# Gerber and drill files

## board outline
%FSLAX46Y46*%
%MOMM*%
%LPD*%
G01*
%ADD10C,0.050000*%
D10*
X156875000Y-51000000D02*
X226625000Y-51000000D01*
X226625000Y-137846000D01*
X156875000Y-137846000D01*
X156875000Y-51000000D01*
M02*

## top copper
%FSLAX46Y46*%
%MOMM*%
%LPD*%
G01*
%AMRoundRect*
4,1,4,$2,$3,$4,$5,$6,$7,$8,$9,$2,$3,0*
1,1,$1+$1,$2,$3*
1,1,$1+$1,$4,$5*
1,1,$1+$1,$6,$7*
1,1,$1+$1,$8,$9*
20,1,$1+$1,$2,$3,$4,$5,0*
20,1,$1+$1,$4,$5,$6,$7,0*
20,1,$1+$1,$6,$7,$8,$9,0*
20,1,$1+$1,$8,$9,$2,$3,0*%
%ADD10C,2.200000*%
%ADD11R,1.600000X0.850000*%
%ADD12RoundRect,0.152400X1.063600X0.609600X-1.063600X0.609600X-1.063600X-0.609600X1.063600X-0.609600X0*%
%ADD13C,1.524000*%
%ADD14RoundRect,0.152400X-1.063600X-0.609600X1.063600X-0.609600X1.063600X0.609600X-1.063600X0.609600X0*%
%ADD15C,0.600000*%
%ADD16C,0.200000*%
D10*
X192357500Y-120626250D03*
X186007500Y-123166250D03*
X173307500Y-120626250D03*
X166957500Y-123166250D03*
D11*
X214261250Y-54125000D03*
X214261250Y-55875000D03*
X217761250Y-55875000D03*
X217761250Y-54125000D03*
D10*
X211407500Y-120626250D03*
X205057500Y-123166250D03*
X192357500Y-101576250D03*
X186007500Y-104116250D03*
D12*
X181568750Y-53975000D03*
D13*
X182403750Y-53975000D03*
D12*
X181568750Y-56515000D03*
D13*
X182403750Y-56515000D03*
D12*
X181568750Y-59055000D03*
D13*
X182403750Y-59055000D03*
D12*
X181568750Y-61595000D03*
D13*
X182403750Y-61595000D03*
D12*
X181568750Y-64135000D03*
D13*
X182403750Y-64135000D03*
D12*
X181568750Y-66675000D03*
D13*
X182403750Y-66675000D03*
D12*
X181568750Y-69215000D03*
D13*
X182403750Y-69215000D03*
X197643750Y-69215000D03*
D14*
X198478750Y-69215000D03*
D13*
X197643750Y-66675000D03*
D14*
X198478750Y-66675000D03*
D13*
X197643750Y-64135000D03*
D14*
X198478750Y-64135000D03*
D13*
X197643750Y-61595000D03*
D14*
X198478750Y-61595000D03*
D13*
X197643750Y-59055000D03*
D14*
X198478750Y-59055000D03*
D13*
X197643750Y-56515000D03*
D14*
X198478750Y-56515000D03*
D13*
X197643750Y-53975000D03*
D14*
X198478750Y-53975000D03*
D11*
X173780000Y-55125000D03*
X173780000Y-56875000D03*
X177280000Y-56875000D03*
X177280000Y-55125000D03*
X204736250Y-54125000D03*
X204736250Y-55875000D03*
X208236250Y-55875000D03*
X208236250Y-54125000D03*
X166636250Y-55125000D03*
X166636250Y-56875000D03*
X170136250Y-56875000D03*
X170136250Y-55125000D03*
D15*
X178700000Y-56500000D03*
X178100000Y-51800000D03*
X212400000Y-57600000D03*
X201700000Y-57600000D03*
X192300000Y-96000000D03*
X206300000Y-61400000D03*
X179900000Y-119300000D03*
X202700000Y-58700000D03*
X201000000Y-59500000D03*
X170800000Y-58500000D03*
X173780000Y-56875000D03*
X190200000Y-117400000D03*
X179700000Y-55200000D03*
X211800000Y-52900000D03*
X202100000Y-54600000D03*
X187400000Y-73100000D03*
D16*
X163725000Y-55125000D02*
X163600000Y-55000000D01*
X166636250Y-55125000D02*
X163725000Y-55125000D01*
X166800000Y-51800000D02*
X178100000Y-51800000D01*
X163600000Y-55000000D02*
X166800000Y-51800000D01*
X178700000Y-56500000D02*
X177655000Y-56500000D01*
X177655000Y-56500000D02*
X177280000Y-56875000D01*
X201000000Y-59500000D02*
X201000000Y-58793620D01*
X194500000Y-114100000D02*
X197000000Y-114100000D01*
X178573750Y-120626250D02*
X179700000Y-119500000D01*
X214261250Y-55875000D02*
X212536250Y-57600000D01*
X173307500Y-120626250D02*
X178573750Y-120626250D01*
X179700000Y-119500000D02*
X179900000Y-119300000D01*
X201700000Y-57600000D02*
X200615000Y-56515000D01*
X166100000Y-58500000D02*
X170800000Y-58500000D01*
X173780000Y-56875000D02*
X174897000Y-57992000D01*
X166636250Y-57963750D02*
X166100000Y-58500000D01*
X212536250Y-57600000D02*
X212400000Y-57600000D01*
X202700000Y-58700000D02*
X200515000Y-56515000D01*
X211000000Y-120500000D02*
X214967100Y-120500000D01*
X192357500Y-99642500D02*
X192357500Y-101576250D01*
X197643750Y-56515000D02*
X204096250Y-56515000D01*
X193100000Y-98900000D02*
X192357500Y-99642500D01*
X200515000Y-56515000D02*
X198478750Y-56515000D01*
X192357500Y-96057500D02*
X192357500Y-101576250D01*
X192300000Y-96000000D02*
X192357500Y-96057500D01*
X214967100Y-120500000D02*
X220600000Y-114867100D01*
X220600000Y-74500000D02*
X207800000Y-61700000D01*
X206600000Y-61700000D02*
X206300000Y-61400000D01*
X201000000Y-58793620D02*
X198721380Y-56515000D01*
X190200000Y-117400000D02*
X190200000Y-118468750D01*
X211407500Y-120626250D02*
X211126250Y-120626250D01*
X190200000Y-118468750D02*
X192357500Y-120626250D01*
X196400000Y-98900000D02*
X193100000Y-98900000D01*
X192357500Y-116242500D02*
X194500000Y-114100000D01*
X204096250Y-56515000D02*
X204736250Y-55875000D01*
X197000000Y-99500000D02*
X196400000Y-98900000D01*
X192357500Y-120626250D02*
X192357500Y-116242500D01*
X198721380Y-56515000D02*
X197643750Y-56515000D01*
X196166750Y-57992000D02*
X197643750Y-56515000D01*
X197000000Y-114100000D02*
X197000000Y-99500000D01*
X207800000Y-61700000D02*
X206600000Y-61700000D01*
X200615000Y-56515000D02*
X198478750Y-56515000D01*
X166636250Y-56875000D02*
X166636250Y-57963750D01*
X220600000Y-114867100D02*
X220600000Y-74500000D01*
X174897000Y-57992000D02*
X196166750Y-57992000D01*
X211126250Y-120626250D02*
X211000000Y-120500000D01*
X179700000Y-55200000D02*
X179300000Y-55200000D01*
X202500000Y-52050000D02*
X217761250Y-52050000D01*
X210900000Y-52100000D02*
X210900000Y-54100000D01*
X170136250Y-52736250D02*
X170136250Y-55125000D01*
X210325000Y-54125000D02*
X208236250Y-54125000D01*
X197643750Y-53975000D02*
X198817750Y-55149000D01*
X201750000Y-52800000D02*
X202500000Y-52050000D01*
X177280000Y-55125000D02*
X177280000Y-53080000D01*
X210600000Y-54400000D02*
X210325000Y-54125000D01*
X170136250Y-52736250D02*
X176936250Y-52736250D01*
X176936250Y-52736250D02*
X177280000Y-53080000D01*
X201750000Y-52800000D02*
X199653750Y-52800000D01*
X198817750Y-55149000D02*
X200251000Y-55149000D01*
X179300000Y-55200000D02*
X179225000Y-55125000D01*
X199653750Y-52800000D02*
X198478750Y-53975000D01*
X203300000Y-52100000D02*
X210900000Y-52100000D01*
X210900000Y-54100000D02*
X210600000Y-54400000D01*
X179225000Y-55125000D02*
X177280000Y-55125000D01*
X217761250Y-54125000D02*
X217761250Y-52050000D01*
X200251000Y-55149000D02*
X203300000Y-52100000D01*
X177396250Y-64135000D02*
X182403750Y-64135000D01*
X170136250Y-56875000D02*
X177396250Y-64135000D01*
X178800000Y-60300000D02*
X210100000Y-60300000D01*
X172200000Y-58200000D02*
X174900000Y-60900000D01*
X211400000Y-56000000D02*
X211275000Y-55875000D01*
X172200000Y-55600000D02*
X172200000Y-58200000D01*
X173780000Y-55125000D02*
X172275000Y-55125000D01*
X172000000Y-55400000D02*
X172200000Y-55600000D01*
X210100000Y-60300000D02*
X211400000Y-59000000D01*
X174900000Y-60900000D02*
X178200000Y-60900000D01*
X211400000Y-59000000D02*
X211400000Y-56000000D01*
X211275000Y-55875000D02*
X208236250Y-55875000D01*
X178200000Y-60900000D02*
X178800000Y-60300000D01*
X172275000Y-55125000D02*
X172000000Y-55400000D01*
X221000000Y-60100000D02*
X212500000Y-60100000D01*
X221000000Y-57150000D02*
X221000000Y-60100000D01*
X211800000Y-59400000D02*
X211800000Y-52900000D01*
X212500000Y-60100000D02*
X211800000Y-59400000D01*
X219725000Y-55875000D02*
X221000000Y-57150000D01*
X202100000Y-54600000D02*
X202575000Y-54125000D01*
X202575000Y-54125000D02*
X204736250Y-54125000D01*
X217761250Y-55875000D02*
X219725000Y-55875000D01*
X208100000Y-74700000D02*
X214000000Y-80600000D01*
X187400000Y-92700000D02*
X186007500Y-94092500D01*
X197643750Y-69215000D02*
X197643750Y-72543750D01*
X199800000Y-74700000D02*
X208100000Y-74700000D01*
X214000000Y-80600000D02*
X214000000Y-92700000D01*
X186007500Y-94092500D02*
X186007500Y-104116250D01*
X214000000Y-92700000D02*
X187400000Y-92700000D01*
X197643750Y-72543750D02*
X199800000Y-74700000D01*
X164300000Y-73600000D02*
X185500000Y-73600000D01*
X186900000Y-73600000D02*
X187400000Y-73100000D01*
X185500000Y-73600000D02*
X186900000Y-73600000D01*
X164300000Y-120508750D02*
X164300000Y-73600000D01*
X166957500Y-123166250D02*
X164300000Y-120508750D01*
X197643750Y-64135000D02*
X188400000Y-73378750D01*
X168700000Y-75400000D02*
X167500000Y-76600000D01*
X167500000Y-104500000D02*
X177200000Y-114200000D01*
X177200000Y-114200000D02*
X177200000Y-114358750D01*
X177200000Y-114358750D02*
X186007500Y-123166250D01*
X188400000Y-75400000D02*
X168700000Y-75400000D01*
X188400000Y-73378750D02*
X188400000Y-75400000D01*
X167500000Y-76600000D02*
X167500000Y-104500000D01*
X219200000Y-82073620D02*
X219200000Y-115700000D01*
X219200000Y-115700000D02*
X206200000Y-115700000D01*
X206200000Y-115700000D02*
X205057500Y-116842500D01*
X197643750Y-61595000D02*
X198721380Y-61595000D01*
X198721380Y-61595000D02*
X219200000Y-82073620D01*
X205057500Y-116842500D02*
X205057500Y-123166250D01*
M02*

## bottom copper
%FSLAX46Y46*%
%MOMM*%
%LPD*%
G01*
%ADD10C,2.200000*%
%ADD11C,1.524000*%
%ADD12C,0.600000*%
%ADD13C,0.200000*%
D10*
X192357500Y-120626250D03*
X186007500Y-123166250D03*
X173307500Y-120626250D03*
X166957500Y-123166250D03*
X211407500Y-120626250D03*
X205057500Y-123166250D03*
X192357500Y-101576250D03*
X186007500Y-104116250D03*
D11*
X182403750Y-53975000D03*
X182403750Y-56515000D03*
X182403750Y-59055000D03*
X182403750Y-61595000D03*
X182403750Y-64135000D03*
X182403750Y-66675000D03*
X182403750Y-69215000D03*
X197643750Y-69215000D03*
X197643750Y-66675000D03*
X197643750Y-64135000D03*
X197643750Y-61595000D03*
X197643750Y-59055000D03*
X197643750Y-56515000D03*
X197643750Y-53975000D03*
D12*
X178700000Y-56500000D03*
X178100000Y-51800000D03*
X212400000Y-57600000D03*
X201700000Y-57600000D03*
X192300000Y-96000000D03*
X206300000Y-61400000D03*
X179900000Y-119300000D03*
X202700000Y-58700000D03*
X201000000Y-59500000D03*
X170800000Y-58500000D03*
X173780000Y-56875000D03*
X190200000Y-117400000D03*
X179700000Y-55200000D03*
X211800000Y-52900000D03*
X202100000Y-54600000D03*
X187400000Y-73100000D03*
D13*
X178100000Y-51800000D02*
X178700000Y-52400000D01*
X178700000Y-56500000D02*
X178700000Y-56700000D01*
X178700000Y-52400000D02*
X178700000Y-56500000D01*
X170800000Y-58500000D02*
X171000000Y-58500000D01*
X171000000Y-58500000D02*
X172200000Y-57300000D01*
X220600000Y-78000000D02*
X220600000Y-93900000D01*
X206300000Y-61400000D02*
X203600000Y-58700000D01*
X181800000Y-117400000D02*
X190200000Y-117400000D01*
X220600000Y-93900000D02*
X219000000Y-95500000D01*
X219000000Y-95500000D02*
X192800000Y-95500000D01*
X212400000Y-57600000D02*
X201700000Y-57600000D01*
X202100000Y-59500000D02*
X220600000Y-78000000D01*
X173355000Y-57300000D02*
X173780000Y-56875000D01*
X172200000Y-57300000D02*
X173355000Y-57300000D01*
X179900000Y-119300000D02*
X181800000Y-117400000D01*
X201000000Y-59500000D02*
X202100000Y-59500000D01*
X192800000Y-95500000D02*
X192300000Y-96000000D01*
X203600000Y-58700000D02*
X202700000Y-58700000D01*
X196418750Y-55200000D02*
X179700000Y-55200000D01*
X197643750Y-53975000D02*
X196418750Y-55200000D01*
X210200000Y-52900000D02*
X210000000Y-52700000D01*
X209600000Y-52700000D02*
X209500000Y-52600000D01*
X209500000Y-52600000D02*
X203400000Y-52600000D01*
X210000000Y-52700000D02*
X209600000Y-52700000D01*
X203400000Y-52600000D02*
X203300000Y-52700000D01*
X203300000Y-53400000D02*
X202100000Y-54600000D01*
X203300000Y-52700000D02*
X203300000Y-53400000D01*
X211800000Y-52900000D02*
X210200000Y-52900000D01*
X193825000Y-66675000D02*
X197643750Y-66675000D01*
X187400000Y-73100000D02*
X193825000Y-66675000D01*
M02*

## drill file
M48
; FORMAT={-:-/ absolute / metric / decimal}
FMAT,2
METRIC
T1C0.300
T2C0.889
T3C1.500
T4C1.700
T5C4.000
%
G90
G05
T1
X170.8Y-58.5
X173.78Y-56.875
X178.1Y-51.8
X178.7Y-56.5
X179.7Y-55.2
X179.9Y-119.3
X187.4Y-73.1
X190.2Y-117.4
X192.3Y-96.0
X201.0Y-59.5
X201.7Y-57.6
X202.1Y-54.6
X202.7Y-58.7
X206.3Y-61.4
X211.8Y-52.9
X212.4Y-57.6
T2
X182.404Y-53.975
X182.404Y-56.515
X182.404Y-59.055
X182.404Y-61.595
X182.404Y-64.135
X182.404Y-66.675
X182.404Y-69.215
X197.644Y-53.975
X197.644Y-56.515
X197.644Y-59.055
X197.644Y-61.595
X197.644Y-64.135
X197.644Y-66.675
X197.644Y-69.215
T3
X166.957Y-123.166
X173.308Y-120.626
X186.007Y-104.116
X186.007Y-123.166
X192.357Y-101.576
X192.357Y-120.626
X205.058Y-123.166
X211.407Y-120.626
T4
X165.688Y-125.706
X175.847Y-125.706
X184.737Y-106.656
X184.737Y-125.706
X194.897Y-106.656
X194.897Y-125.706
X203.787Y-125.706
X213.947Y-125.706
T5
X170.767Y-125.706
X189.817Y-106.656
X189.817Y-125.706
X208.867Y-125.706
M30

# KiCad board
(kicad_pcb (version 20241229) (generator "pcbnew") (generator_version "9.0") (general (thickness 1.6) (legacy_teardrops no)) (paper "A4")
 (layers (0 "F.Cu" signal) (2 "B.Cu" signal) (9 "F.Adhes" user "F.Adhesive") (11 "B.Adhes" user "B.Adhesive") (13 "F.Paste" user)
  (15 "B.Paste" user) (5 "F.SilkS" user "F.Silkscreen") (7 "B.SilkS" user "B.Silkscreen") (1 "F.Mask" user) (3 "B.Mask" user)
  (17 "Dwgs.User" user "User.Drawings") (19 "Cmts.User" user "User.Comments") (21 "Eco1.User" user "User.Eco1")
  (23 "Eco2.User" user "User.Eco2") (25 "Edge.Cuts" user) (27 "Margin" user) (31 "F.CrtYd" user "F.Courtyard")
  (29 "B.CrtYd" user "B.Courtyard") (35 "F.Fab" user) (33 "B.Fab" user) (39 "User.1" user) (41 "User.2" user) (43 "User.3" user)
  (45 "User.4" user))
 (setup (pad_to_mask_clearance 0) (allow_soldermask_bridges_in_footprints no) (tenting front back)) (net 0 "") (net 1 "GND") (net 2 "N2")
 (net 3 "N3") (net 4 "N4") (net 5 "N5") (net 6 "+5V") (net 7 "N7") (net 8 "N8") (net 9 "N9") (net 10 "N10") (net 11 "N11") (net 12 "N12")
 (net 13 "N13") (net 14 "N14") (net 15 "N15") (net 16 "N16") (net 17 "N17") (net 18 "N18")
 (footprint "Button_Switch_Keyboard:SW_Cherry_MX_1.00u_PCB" (layer "F.Cu") (at 192.3575 120.62625)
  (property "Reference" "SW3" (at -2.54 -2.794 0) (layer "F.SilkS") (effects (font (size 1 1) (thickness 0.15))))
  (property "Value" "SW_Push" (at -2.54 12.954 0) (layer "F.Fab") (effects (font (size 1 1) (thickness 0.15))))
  (pad "" np_thru_hole circle (at -7.62 5.08) (size 1.7 1.7) (drill 1.7) (layers "*.Cu" "*.Mask"))
  (pad "" np_thru_hole circle (at -2.54 5.08) (size 4 4) (drill 4) (layers "*.Cu" "*.Mask"))
  (pad "" np_thru_hole circle (at 2.54 5.08) (size 1.7 1.7) (drill 1.7) (layers "*.Cu" "*.Mask"))
  (pad "1" thru_hole circle (at 0 0) (size 2.2 2.2) (drill 1.5) (layers "*.Cu" "*.Mask") (remove_unused_layers no) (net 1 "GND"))
  (pad "2" thru_hole circle (at -6.35 2.54) (size 2.2 2.2) (drill 1.5) (layers "*.Cu" "*.Mask") (remove_unused_layers no) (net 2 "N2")))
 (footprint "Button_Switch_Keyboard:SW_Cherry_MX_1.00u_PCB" (layer "F.Cu") (at 173.3075 120.62625)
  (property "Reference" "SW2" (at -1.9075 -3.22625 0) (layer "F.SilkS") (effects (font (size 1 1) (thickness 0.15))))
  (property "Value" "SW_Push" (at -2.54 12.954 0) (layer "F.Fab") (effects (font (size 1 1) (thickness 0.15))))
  (pad "" np_thru_hole circle (at -7.62 5.08) (size 1.7 1.7) (drill 1.7) (layers "*.Cu" "*.Mask"))
  (pad "" np_thru_hole circle (at -2.54 5.08) (size 4 4) (drill 4) (layers "*.Cu" "*.Mask"))
  (pad "" np_thru_hole circle (at 2.54 5.08) (size 1.7 1.7) (drill 1.7) (layers "*.Cu" "*.Mask"))
  (pad "1" thru_hole circle (at 0 0) (size 2.2 2.2) (drill 1.5) (layers "*.Cu" "*.Mask") (remove_unused_layers no) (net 1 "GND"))
  (pad "2" thru_hole circle (at -6.35 2.54) (size 2.2 2.2) (drill 1.5) (layers "*.Cu" "*.Mask") (remove_unused_layers no) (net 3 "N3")))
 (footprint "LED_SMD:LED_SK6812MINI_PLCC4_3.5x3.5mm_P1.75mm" (layer "F.Cu") (at 216.01125 55)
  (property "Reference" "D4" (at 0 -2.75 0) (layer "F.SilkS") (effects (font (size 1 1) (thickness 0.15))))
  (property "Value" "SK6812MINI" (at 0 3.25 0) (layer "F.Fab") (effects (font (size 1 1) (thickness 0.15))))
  (pad "1" smd rect (at -1.75 -0.875) (size 1.6 0.85) (layers "F.Cu" "F.Mask" "F.Paste") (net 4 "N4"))
  (pad "2" smd rect (at -1.75 0.875) (size 1.6 0.85) (layers "F.Cu" "F.Mask" "F.Paste") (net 1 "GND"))
  (pad "3" smd rect (at 1.75 0.875) (size 1.6 0.85) (layers "F.Cu" "F.Mask" "F.Paste") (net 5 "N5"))
  (pad "4" smd rect (at 1.75 -0.875) (size 1.6 0.85) (layers "F.Cu" "F.Mask" "F.Paste") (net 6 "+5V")))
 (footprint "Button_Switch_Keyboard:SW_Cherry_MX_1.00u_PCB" (layer "F.Cu") (at 211.4075 120.62625)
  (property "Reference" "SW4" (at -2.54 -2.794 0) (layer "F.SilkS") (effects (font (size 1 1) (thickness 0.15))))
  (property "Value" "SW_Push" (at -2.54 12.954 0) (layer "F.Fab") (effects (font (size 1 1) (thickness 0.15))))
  (pad "" np_thru_hole circle (at -7.62 5.08) (size 1.7 1.7) (drill 1.7) (layers "*.Cu" "*.Mask"))
  (pad "" np_thru_hole circle (at -2.54 5.08) (size 4 4) (drill 4) (layers "*.Cu" "*.Mask"))
  (pad "" np_thru_hole circle (at 2.54 5.08) (size 1.7 1.7) (drill 1.7) (layers "*.Cu" "*.Mask"))
  (pad "1" thru_hole circle (at 0 0) (size 2.2 2.2) (drill 1.5) (layers "*.Cu" "*.Mask") (remove_unused_layers no) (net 1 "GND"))
  (pad "2" thru_hole circle (at -6.35 2.54) (size 2.2 2.2) (drill 1.5) (layers "*.Cu" "*.Mask") (remove_unused_layers no) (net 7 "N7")))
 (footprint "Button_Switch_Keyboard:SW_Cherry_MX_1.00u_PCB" (layer "F.Cu") (at 192.3575 101.57625)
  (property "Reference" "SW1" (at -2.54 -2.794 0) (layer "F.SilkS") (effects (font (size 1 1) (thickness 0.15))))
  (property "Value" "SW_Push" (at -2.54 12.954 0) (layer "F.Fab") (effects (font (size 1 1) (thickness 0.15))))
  (pad "" np_thru_hole circle (at -7.62 5.08) (size 1.7 1.7) (drill 1.7) (layers "*.Cu" "*.Mask"))
  (pad "" np_thru_hole circle (at -2.54 5.08) (size 4 4) (drill 4) (layers "*.Cu" "*.Mask"))
  (pad "" np_thru_hole circle (at 2.54 5.08) (size 1.7 1.7) (drill 1.7) (layers "*.Cu" "*.Mask"))
  (pad "1" thru_hole circle (at 0 0) (size 2.2 2.2) (drill 1.5) (layers "*.Cu" "*.Mask") (remove_unused_layers no) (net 1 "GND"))
  (pad "2" thru_hole circle (at -6.35 2.54) (size 2.2 2.2) (drill 1.5) (layers "*.Cu" "*.Mask") (remove_unused_layers no) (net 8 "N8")))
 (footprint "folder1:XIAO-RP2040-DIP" (layer "F.Cu") (at 190.02375 61.595)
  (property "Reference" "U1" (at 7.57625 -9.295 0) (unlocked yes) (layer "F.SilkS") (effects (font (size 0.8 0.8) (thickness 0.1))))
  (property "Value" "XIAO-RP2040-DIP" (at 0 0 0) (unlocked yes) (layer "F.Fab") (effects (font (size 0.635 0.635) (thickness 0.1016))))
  (pad "1" smd roundrect (at -8.455 -7.62 180) (size 2.432 1.524) (layers "F.Cu" "F.Mask") (roundrect_rratio 0.1) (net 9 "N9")
   (thermal_bridge_angle 45))
  (pad "1" thru_hole circle (at -7.62 -7.62 180) (size 1.524 1.524) (drill 0.889) (layers "*.Cu" "*.Mask") (remove_unused_layers no)
   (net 9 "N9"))
  (pad "2" smd roundrect (at -8.455 -5.08 180) (size 2.432 1.524) (layers "F.Cu" "F.Mask") (roundrect_rratio 0.1) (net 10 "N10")
   (thermal_bridge_angle 45))
  (pad "2" thru_hole circle (at -7.62 -5.08 180) (size 1.524 1.524) (drill 0.889) (layers "*.Cu" "*.Mask") (remove_unused_layers no)
   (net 10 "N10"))
  (pad "3" smd roundrect (at -8.455 -2.54 180) (size 2.432 1.524) (layers "F.Cu" "F.Mask") (roundrect_rratio 0.1) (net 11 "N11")
   (thermal_bridge_angle 45))
  (pad "3" thru_hole circle (at -7.62 -2.54 180) (size 1.524 1.524) (drill 0.889) (layers "*.Cu" "*.Mask") (remove_unused_layers no)
   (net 11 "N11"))
  (pad "4" smd roundrect (at -8.455 0 180) (size 2.432 1.524) (layers "F.Cu" "F.Mask") (roundrect_rratio 0.1) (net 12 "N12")
   (thermal_bridge_angle 45))
  (pad "4" thru_hole circle (at -7.62 0 180) (size 1.524 1.524) (drill 0.889) (layers "*.Cu" "*.Mask") (remove_unused_layers no)
   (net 12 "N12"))
  (pad "5" smd roundrect (at -8.455 2.54 180) (size 2.432 1.524) (layers "F.Cu" "F.Mask") (roundrect_rratio 0.1) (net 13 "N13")
   (thermal_bridge_angle 45))
  (pad "5" thru_hole circle (at -7.62 2.54 180) (size 1.524 1.524) (drill 0.889) (layers "*.Cu" "*.Mask") (remove_unused_layers no)
   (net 13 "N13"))
  (pad "6" smd roundrect (at -8.455 5.08 180) (size 2.432 1.524) (layers "F.Cu" "F.Mask") (roundrect_rratio 0.1) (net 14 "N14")
   (thermal_bridge_angle 45))
  (pad "6" thru_hole circle (at -7.62 5.08 180) (size 1.524 1.524) (drill 0.889) (layers "*.Cu" "*.Mask") (remove_unused_layers no)
   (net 14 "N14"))
  (pad "7" smd roundrect (at -8.455 7.62 180) (size 2.432 1.524) (layers "F.Cu" "F.Mask") (roundrect_rratio 0.1) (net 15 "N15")
   (thermal_bridge_angle 45))
  (pad "7" thru_hole circle (at -7.62 7.62 180) (size 1.524 1.524) (drill 0.889) (layers "*.Cu" "*.Mask") (remove_unused_layers no)
   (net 15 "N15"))
  (pad "8" thru_hole circle (at 7.62 7.62) (size 1.524 1.524) (drill 0.889) (layers "*.Cu" "*.Mask") (remove_unused_layers no) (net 8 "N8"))
  (pad "8" smd roundrect (at 8.455 7.62) (size 2.432 1.524) (layers "F.Cu" "F.Mask") (roundrect_rratio 0.1) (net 8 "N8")
   (thermal_bridge_angle 45))
  (pad "9" thru_hole circle (at 7.62 5.08) (size 1.524 1.524) (drill 0.889) (layers "*.Cu" "*.Mask") (remove_unused_layers no) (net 3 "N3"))
  (pad "9" smd roundrect (at 8.455 5.08) (size 2.432 1.524) (layers "F.Cu" "F.Mask") (roundrect_rratio 0.1) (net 3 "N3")
   (thermal_bridge_angle 45))
  (pad "10" thru_hole circle (at 7.62 2.54) (size 1.524 1.524) (drill 0.889) (layers "*.Cu" "*.Mask") (remove_unused_layers no) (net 2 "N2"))
  (pad "10" smd roundrect (at 8.455 2.54) (size 2.432 1.524) (layers "F.Cu" "F.Mask") (roundrect_rratio 0.1) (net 2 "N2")
   (thermal_bridge_angle 45))
  (pad "11" thru_hole circle (at 7.62 0) (size 1.524 1.524) (drill 0.889) (layers "*.Cu" "*.Mask") (remove_unused_layers no) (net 7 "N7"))
  (pad "11" smd roundrect (at 8.455 0) (size 2.432 1.524) (layers "F.Cu" "F.Mask") (roundrect_rratio 0.1) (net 7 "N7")
   (thermal_bridge_angle 45))
  (pad "12" thru_hole circle (at 7.62 -2.54) (size 1.524 1.524) (drill 0.889) (layers "*.Cu" "*.Mask") (remove_unused_layers no)
   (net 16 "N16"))
  (pad "12" smd roundrect (at 8.455 -2.54) (size 2.432 1.524) (layers "F.Cu" "F.Mask") (roundrect_rratio 0.1) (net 16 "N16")
   (thermal_bridge_angle 45))
  (pad "13" thru_hole circle (at 7.62 -5.08) (size 1.524 1.524) (drill 0.889) (layers "*.Cu" "*.Mask") (remove_unused_layers no)
   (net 1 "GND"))
  (pad "13" smd roundrect (at 8.455 -5.08) (size 2.432 1.524) (layers "F.Cu" "F.Mask") (roundrect_rratio 0.1) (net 1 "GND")
   (thermal_bridge_angle 45))
  (pad "14" thru_hole circle (at 7.62 -7.62) (size 1.524 1.524) (drill 0.889) (layers "*.Cu" "*.Mask") (remove_unused_layers no)
   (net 6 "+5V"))
  (pad "14" smd roundrect (at 8.455 -7.62) (size 2.432 1.524) (layers "F.Cu" "F.Mask") (roundrect_rratio 0.1) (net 6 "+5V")
   (thermal_bridge_angle 45)))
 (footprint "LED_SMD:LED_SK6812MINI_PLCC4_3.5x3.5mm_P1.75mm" (layer "F.Cu") (at 175.53 56)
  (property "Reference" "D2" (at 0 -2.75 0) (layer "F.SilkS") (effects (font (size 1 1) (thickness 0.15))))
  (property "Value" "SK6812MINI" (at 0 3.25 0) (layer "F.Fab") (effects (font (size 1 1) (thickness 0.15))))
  (pad "1" smd rect (at -1.75 -0.875) (size 1.6 0.85) (layers "F.Cu" "F.Mask" "F.Paste") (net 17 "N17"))
  (pad "2" smd rect (at -1.75 0.875) (size 1.6 0.85) (layers "F.Cu" "F.Mask" "F.Paste") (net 1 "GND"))
  (pad "3" smd rect (at 1.75 0.875) (size 1.6 0.85) (layers "F.Cu" "F.Mask" "F.Paste") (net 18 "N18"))
  (pad "4" smd rect (at 1.75 -0.875) (size 1.6 0.85) (layers "F.Cu" "F.Mask" "F.Paste") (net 6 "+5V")))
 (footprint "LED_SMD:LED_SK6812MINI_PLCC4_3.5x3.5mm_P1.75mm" (layer "F.Cu") (at 206.48625 55)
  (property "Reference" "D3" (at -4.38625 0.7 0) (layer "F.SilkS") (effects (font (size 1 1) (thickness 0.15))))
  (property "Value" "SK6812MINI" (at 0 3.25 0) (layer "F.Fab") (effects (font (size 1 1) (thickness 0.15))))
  (pad "1" smd rect (at -1.75 -0.875) (size 1.6 0.85) (layers "F.Cu" "F.Mask" "F.Paste") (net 5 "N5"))
  (pad "2" smd rect (at -1.75 0.875) (size 1.6 0.85) (layers "F.Cu" "F.Mask" "F.Paste") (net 1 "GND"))
  (pad "3" smd rect (at 1.75 0.875) (size 1.6 0.85) (layers "F.Cu" "F.Mask" "F.Paste") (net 17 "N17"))
  (pad "4" smd rect (at 1.75 -0.875) (size 1.6 0.85) (layers "F.Cu" "F.Mask" "F.Paste") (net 6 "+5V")))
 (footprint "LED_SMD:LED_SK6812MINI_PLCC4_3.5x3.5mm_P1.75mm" (layer "F.Cu") (at 168.38625 56)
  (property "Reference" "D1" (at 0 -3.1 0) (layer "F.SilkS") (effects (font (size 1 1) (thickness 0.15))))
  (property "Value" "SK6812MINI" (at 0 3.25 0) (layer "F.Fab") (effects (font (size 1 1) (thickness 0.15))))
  (pad "1" smd rect (at -1.75 -0.875) (size 1.6 0.85) (layers "F.Cu" "F.Mask" "F.Paste") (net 18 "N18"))
  (pad "2" smd rect (at -1.75 0.875) (size 1.6 0.85) (layers "F.Cu" "F.Mask" "F.Paste") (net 1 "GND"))
  (pad "3" smd rect (at 1.75 0.875) (size 1.6 0.85) (layers "F.Cu" "F.Mask" "F.Paste") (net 13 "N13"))
  (pad "4" smd rect (at 1.75 -0.875) (size 1.6 0.85) (layers "F.Cu" "F.Mask" "F.Paste") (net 6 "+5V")))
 (gr_rect (start 156.875 51) (end 226.625 137.846) (stroke (width 0.05) (type default)) (fill no) (layer "Edge.Cuts"))
 (segment (start 163.725 55.125) (end 163.6 55) (width 0.2) (layer "F.Cu") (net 18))
 (segment (start 166.63625 55.125) (end 163.725 55.125) (width 0.2) (layer "F.Cu") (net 18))
 (segment (start 166.8 51.8) (end 178.1 51.8) (width 0.2) (layer "F.Cu") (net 18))
 (segment (start 163.6 55) (end 166.8 51.8) (width 0.2) (layer "F.Cu") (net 18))
 (segment (start 178.7 56.5) (end 177.655 56.5) (width 0.2) (layer "F.Cu") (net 18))
 (segment (start 177.655 56.5) (end 177.28 56.875) (width 0.2) (layer "F.Cu") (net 18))
 (via (at 178.7 56.5) (size 0.6) (drill 0.3) (layers "F.Cu" "B.Cu") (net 18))
 (via (at 178.1 51.8) (size 0.6) (drill 0.3) (layers "F.Cu" "B.Cu") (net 18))
 (segment (start 178.1 51.8) (end 178.7 52.4) (width 0.2) (layer "B.Cu") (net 18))
 (segment (start 178.7 56.5) (end 178.7 56.7) (width 0.2) (layer "B.Cu") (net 18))
 (segment (start 178.7 52.4) (end 178.7 56.5) (width 0.2) (layer "B.Cu") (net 18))
 (segment (start 201 59.5) (end 201 58.79362) (width 0.2) (layer "F.Cu") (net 1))
 (segment (start 194.5 114.1) (end 197 114.1) (width 0.2) (layer "F.Cu") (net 1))
 (segment (start 178.57375 120.62625) (end 179.7 119.5) (width 0.2) (layer "F.Cu") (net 1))
 (segment (start 214.26125 55.875) (end 212.53625 57.6) (width 0.2) (layer "F.Cu") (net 1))
 (segment (start 173.3075 120.62625) (end 178.57375 120.62625) (width 0.2) (layer "F.Cu") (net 1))
 (segment (start 179.7 119.5) (end 179.9 119.3) (width 0.2) (layer "F.Cu") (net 1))
 (segment (start 201.7 57.6) (end 200.615 56.515) (width 0.2) (layer "F.Cu") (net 1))
 (segment (start 166.1 58.5) (end 170.8 58.5) (width 0.2) (layer "F.Cu") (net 1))
 (segment (start 173.78 56.875) (end 174.897 57.992) (width 0.2) (layer "F.Cu") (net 1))
 (segment (start 166.63625 57.96375) (end 166.1 58.5) (width 0.2) (layer "F.Cu") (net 1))
 (segment (start 212.53625 57.6) (end 212.4 57.6) (width 0.2) (layer "F.Cu") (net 1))
 (segment (start 202.7 58.7) (end 200.515 56.515) (width 0.2) (layer "F.Cu") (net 1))
 (segment (start 211 120.5) (end 214.9671 120.5) (width 0.2) (layer "F.Cu") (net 1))
 (segment (start 192.3575 99.6425) (end 192.3575 101.57625) (width 0.2) (layer "F.Cu") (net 1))
 (segment (start 197.64375 56.515) (end 204.09625 56.515) (width 0.2) (layer "F.Cu") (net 1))
 (segment (start 193.1 98.9) (end 192.3575 99.6425) (width 0.2) (layer "F.Cu") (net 1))
 (segment (start 200.515 56.515) (end 198.47875 56.515) (width 0.2) (layer "F.Cu") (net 1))
 (segment (start 192.3575 96.0575) (end 192.3575 101.57625) (width 0.2) (layer "F.Cu") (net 1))
 (segment (start 192.3 96) (end 192.3575 96.0575) (width 0.2) (layer "F.Cu") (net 1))
 (segment (start 214.9671 120.5) (end 220.6 114.8671) (width 0.2) (layer "F.Cu") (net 1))
 (segment (start 220.6 74.5) (end 207.8 61.7) (width 0.2) (layer "F.Cu") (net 1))
 (segment (start 206.6 61.7) (end 206.3 61.4) (width 0.2) (layer "F.Cu") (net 1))
 (segment (start 201 58.79362) (end 198.72138 56.515) (width 0.2) (layer "F.Cu") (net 1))
 (segment (start 190.2 117.4) (end 190.2 118.46875) (width 0.2) (layer "F.Cu") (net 1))
 (segment (start 211.4075 120.62625) (end 211.12625 120.62625) (width 0.2) (layer "F.Cu") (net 1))
 (segment (start 190.2 118.46875) (end 192.3575 120.62625) (width 0.2) (layer "F.Cu") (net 1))
 (segment (start 196.4 98.9) (end 193.1 98.9) (width 0.2) (layer "F.Cu") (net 1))
 (segment (start 192.3575 116.2425) (end 194.5 114.1) (width 0.2) (layer "F.Cu") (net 1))
 (segment (start 204.09625 56.515) (end 204.73625 55.875) (width 0.2) (layer "F.Cu") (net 1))
 (segment (start 197 99.5) (end 196.4 98.9) (width 0.2) (layer "F.Cu") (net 1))
 (segment (start 192.3575 120.62625) (end 192.3575 116.2425) (width 0.2) (layer "F.Cu") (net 1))
 (segment (start 198.72138 56.515) (end 197.64375 56.515) (width 0.2) (layer "F.Cu") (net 1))
 (segment (start 196.16675 57.992) (end 197.64375 56.515) (width 0.2) (layer "F.Cu") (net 1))
 (segment (start 197 114.1) (end 197 99.5) (width 0.2) (layer "F.Cu") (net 1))
 (segment (start 207.8 61.7) (end 206.6 61.7) (width 0.2) (layer "F.Cu") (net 1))
 (segment (start 200.615 56.515) (end 198.47875 56.515) (width 0.2) (layer "F.Cu") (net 1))
 (segment (start 166.63625 56.875) (end 166.63625 57.96375) (width 0.2) (layer "F.Cu") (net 1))
 (segment (start 220.6 114.8671) (end 220.6 74.5) (width 0.2) (layer "F.Cu") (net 1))
 (segment (start 174.897 57.992) (end 196.16675 57.992) (width 0.2) (layer "F.Cu") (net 1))
 (segment (start 211.12625 120.62625) (end 211 120.5) (width 0.2) (layer "F.Cu") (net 1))
 (via (at 212.4 57.6) (size 0.6) (drill 0.3) (layers "F.Cu" "B.Cu") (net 1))
 (via (at 201.7 57.6) (size 0.6) (drill 0.3) (layers "F.Cu" "B.Cu") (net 1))
 (via (at 192.3 96) (size 0.6) (drill 0.3) (layers "F.Cu" "B.Cu") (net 1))
 (via (at 206.3 61.4) (size 0.6) (drill 0.3) (layers "F.Cu" "B.Cu") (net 1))
 (via (at 179.9 119.3) (size 0.6) (drill 0.3) (layers "F.Cu" "B.Cu") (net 1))
 (via (at 202.7 58.7) (size 0.6) (drill 0.3) (layers "F.Cu" "B.Cu") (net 1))
 (via (at 201 59.5) (size 0.6) (drill 0.3) (layers "F.Cu" "B.Cu") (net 1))
 (via (at 170.8 58.5) (size 0.6) (drill 0.3) (layers "F.Cu" "B.Cu") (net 1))
 (via (at 173.78 56.875) (size 0.6) (drill 0.3) (layers "F.Cu" "B.Cu") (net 1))
 (via (at 190.2 117.4) (size 0.6) (drill 0.3) (layers "F.Cu" "B.Cu") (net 1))
 (segment (start 170.8 58.5) (end 171 58.5) (width 0.2) (layer "B.Cu") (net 1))
 (segment (start 171 58.5) (end 172.2 57.3) (width 0.2) (layer "B.Cu") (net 1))
 (segment (start 220.6 78) (end 220.6 93.9) (width 0.2) (layer "B.Cu") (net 1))
 (segment (start 206.3 61.4) (end 203.6 58.7) (width 0.2) (layer "B.Cu") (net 1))
 (segment (start 181.8 117.4) (end 190.2 117.4) (width 0.2) (layer "B.Cu") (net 1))
 (segment (start 220.6 93.9) (end 219 95.5) (width 0.2) (layer "B.Cu") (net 1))
 (segment (start 219 95.5) (end 192.8 95.5) (width 0.2) (layer "B.Cu") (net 1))
 (segment (start 212.4 57.6) (end 201.7 57.6) (width 0.2) (layer "B.Cu") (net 1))
 (segment (start 202.1 59.5) (end 220.6 78) (width 0.2) (layer "B.Cu") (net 1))
 (segment (start 173.355 57.3) (end 173.78 56.875) (width 0.2) (layer "B.Cu") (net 1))
 (segment (start 172.2 57.3) (end 173.355 57.3) (width 0.2) (layer "B.Cu") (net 1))
 (segment (start 179.9 119.3) (end 181.8 117.4) (width 0.2) (layer "B.Cu") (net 1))
 (segment (start 201 59.5) (end 202.1 59.5) (width 0.2) (layer "B.Cu") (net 1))
 (segment (start 192.8 95.5) (end 192.3 96) (width 0.2) (layer "B.Cu") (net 1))
 (segment (start 203.6 58.7) (end 202.7 58.7) (width 0.2) (layer "B.Cu") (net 1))
 (segment (start 179.7 55.2) (end 179.3 55.2) (width 0.2) (layer "F.Cu") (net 6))
 (segment (start 202.5 52.05) (end 217.76125 52.05) (width 0.2) (layer "F.Cu") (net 6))
 (segment (start 210.9 52.1) (end 210.9 54.1) (width 0.2) (layer "F.Cu") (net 6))
 (segment (start 170.13625 52.73625) (end 170.13625 55.125) (width 0.2) (layer "F.Cu") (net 6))
 (segment (start 210.325 54.125) (end 208.23625 54.125) (width 0.2) (layer "F.Cu") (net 6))
 (segment (start 197.64375 53.975) (end 198.81775 55.149) (width 0.2) (layer "F.Cu") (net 6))
 (segment (start 201.75 52.8) (end 202.5 52.05) (width 0.2) (layer "F.Cu") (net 6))
 (segment (start 177.28 55.125) (end 177.28 53.08) (width 0.2) (layer "F.Cu") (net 6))
 (segment (start 210.6 54.4) (end 210.325 54.125) (width 0.2) (layer "F.Cu") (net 6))
 (segment (start 170.13625 52.73625) (end 176.93625 52.73625) (width 0.2) (layer "F.Cu") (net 6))
 (segment (start 176.93625 52.73625) (end 177.28 53.08) (width 0.2) (layer "F.Cu") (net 6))
 (segment (start 201.75 52.8) (end 199.65375 52.8) (width 0.2) (layer "F.Cu") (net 6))
 (segment (start 198.81775 55.149) (end 200.251 55.149) (width 0.2) (layer "F.Cu") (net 6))
 (segment (start 179.3 55.2) (end 179.225 55.125) (width 0.2) (layer "F.Cu") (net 6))
 (segment (start 199.65375 52.8) (end 198.47875 53.975) (width 0.2) (layer "F.Cu") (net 6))
 (segment (start 203.3 52.1) (end 210.9 52.1) (width 0.2) (layer "F.Cu") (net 6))
 (segment (start 210.9 54.1) (end 210.6 54.4) (width 0.2) (layer "F.Cu") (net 6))
 (segment (start 179.225 55.125) (end 177.28 55.125) (width 0.2) (layer "F.Cu") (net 6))
 (segment (start 217.76125 54.125) (end 217.76125 52.05) (width 0.2) (layer "F.Cu") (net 6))
 (segment (start 200.251 55.149) (end 203.3 52.1) (width 0.2) (layer "F.Cu") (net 6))
 (via (at 179.7 55.2) (size 0.6) (drill 0.3) (layers "F.Cu" "B.Cu") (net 6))
 (segment (start 196.41875 55.2) (end 179.7 55.2) (width 0.2) (layer "B.Cu") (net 6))
 (segment (start 197.64375 53.975) (end 196.41875 55.2) (width 0.2) (layer "B.Cu") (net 6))
 (segment (start 177.39625 64.135) (end 182.40375 64.135) (width 0.2) (layer "F.Cu") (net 13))
 (segment (start 170.13625 56.875) (end 177.39625 64.135) (width 0.2) (layer "F.Cu") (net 13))
 (segment (start 178.8 60.3) (end 210.1 60.3) (width 0.2) (layer "F.Cu") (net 17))
 (segment (start 172.2 58.2) (end 174.9 60.9) (width 0.2) (layer "F.Cu") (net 17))
 (segment (start 211.4 56) (end 211.275 55.875) (width 0.2) (layer "F.Cu") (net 17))
 (segment (start 172.2 55.6) (end 172.2 58.2) (width 0.2) (layer "F.Cu") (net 17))
 (segment (start 173.78 55.125) (end 172.275 55.125) (width 0.2) (layer "F.Cu") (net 17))
 (segment (start 172 55.4) (end 172.2 55.6) (width 0.2) (layer "F.Cu") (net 17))
 (segment (start 210.1 60.3) (end 211.4 59) (width 0.2) (layer "F.Cu") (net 17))
 (segment (start 174.9 60.9) (end 178.2 60.9) (width 0.2) (layer "F.Cu") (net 17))
 (segment (start 211.4 59) (end 211.4 56) (width 0.2) (layer "F.Cu") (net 17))
 (segment (start 211.275 55.875) (end 208.23625 55.875) (width 0.2) (layer "F.Cu") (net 17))
 (segment (start 178.2 60.9) (end 178.8 60.3) (width 0.2) (layer "F.Cu") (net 17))
 (segment (start 172.275 55.125) (end 172 55.4) (width 0.2) (layer "F.Cu") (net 17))
 (segment (start 221 60.1) (end 212.5 60.1) (width 0.2) (layer "F.Cu") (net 5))
 (segment (start 221 57.15) (end 221 60.1) (width 0.2) (layer "F.Cu") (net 5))
 (segment (start 211.8 59.4) (end 211.8 52.9) (width 0.2) (layer "F.Cu") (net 5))
 (segment (start 212.5 60.1) (end 211.8 59.4) (width 0.2) (layer "F.Cu") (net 5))
 (segment (start 219.725 55.875) (end 221 57.15) (width 0.2) (layer "F.Cu") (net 5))
 (segment (start 202.1 54.6) (end 202.575 54.125) (width 0.2) (layer "F.Cu") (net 5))
 (segment (start 202.575 54.125) (end 204.73625 54.125) (width 0.2) (layer "F.Cu") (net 5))
 (segment (start 217.76125 55.875) (end 219.725 55.875) (width 0.2) (layer "F.Cu") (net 5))
 (via (at 211.8 52.9) (size 0.6) (drill 0.3) (layers "F.Cu" "B.Cu") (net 5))
 (via (at 202.1 54.6) (size 0.6) (drill 0.3) (layers "F.Cu" "B.Cu") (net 5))
 (segment (start 210.2 52.9) (end 210 52.7) (width 0.2) (layer "B.Cu") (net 5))
 (segment (start 209.6 52.7) (end 209.5 52.6) (width 0.2) (layer "B.Cu") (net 5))
 (segment (start 209.5 52.6) (end 203.4 52.6) (width 0.2) (layer "B.Cu") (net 5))
 (segment (start 210 52.7) (end 209.6 52.7) (width 0.2) (layer "B.Cu") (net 5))
 (segment (start 203.4 52.6) (end 203.3 52.7) (width 0.2) (layer "B.Cu") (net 5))
 (segment (start 203.3 53.4) (end 202.1 54.6) (width 0.2) (layer "B.Cu") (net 5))
 (segment (start 203.3 52.7) (end 203.3 53.4) (width 0.2) (layer "B.Cu") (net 5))
 (segment (start 211.8 52.9) (end 210.2 52.9) (width 0.2) (layer "B.Cu") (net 5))
 (segment (start 208.1 74.7) (end 214 80.6) (width 0.2) (layer "F.Cu") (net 8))
 (segment (start 187.4 92.7) (end 186.0075 94.0925) (width 0.2) (layer "F.Cu") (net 8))
 (segment (start 197.64375 69.215) (end 197.64375 72.54375) (width 0.2) (layer "F.Cu") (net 8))
 (segment (start 199.8 74.7) (end 208.1 74.7) (width 0.2) (layer "F.Cu") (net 8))
 (segment (start 214 80.6) (end 214 92.7) (width 0.2) (layer "F.Cu") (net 8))
 (segment (start 186.0075 94.0925) (end 186.0075 104.11625) (width 0.2) (layer "F.Cu") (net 8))
 (segment (start 214 92.7) (end 187.4 92.7) (width 0.2) (layer "F.Cu") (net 8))
 (segment (start 197.64375 72.54375) (end 199.8 74.7) (width 0.2) (layer "F.Cu") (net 8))
 (segment (start 164.3 73.6) (end 185.5 73.6) (width 0.2) (layer "F.Cu") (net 3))
 (segment (start 186.9 73.6) (end 187.4 73.1) (width 0.2) (layer "F.Cu") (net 3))
 (segment (start 185.5 73.6) (end 186.9 73.6) (width 0.2) (layer "F.Cu") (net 3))
 (segment (start 164.3 120.50875) (end 164.3 73.6) (width 0.2) (layer "F.Cu") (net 3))
 (segment (start 166.9575 123.16625) (end 164.3 120.50875) (width 0.2) (layer "F.Cu") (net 3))
 (via (at 187.4 73.1) (size 0.6) (drill 0.3) (layers "F.Cu" "B.Cu") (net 3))
 (segment (start 193.825 66.675) (end 197.64375 66.675) (width 0.2) (layer "B.Cu") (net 3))
 (segment (start 187.4 73.1) (end 193.825 66.675) (width 0.2) (layer "B.Cu") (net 3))
 (segment (start 197.64375 64.135) (end 188.4 73.37875) (width 0.2) (layer "F.Cu") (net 2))
 (segment (start 168.7 75.4) (end 167.5 76.6) (width 0.2) (layer "F.Cu") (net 2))
 (segment (start 167.5 104.5) (end 177.2 114.2) (width 0.2) (layer "F.Cu") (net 2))
 (segment (start 177.2 114.2) (end 177.2 114.35875) (width 0.2) (layer "F.Cu") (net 2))
 (segment (start 177.2 114.35875) (end 186.0075 123.16625) (width 0.2) (layer "F.Cu") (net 2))
 (segment (start 188.4 75.4) (end 168.7 75.4) (width 0.2) (layer "F.Cu") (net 2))
 (segment (start 188.4 73.37875) (end 188.4 75.4) (width 0.2) (layer "F.Cu") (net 2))
 (segment (start 167.5 76.6) (end 167.5 104.5) (width 0.2) (layer "F.Cu") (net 2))
 (segment (start 219.2 82.07362) (end 219.2 115.7) (width 0.2) (layer "F.Cu") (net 7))
 (segment (start 219.2 115.7) (end 206.2 115.7) (width 0.2) (layer "F.Cu") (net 7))
 (segment (start 206.2 115.7) (end 205.0575 116.8425) (width 0.2) (layer "F.Cu") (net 7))
 (segment (start 197.64375 61.595) (end 198.72138 61.595) (width 0.2) (layer "F.Cu") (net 7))
 (segment (start 198.72138 61.595) (end 219.2 82.07362) (width 0.2) (layer "F.Cu") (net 7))
 (segment (start 205.0575 116.8425) (end 205.0575 123.16625) (width 0.2) (layer "F.Cu") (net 7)))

